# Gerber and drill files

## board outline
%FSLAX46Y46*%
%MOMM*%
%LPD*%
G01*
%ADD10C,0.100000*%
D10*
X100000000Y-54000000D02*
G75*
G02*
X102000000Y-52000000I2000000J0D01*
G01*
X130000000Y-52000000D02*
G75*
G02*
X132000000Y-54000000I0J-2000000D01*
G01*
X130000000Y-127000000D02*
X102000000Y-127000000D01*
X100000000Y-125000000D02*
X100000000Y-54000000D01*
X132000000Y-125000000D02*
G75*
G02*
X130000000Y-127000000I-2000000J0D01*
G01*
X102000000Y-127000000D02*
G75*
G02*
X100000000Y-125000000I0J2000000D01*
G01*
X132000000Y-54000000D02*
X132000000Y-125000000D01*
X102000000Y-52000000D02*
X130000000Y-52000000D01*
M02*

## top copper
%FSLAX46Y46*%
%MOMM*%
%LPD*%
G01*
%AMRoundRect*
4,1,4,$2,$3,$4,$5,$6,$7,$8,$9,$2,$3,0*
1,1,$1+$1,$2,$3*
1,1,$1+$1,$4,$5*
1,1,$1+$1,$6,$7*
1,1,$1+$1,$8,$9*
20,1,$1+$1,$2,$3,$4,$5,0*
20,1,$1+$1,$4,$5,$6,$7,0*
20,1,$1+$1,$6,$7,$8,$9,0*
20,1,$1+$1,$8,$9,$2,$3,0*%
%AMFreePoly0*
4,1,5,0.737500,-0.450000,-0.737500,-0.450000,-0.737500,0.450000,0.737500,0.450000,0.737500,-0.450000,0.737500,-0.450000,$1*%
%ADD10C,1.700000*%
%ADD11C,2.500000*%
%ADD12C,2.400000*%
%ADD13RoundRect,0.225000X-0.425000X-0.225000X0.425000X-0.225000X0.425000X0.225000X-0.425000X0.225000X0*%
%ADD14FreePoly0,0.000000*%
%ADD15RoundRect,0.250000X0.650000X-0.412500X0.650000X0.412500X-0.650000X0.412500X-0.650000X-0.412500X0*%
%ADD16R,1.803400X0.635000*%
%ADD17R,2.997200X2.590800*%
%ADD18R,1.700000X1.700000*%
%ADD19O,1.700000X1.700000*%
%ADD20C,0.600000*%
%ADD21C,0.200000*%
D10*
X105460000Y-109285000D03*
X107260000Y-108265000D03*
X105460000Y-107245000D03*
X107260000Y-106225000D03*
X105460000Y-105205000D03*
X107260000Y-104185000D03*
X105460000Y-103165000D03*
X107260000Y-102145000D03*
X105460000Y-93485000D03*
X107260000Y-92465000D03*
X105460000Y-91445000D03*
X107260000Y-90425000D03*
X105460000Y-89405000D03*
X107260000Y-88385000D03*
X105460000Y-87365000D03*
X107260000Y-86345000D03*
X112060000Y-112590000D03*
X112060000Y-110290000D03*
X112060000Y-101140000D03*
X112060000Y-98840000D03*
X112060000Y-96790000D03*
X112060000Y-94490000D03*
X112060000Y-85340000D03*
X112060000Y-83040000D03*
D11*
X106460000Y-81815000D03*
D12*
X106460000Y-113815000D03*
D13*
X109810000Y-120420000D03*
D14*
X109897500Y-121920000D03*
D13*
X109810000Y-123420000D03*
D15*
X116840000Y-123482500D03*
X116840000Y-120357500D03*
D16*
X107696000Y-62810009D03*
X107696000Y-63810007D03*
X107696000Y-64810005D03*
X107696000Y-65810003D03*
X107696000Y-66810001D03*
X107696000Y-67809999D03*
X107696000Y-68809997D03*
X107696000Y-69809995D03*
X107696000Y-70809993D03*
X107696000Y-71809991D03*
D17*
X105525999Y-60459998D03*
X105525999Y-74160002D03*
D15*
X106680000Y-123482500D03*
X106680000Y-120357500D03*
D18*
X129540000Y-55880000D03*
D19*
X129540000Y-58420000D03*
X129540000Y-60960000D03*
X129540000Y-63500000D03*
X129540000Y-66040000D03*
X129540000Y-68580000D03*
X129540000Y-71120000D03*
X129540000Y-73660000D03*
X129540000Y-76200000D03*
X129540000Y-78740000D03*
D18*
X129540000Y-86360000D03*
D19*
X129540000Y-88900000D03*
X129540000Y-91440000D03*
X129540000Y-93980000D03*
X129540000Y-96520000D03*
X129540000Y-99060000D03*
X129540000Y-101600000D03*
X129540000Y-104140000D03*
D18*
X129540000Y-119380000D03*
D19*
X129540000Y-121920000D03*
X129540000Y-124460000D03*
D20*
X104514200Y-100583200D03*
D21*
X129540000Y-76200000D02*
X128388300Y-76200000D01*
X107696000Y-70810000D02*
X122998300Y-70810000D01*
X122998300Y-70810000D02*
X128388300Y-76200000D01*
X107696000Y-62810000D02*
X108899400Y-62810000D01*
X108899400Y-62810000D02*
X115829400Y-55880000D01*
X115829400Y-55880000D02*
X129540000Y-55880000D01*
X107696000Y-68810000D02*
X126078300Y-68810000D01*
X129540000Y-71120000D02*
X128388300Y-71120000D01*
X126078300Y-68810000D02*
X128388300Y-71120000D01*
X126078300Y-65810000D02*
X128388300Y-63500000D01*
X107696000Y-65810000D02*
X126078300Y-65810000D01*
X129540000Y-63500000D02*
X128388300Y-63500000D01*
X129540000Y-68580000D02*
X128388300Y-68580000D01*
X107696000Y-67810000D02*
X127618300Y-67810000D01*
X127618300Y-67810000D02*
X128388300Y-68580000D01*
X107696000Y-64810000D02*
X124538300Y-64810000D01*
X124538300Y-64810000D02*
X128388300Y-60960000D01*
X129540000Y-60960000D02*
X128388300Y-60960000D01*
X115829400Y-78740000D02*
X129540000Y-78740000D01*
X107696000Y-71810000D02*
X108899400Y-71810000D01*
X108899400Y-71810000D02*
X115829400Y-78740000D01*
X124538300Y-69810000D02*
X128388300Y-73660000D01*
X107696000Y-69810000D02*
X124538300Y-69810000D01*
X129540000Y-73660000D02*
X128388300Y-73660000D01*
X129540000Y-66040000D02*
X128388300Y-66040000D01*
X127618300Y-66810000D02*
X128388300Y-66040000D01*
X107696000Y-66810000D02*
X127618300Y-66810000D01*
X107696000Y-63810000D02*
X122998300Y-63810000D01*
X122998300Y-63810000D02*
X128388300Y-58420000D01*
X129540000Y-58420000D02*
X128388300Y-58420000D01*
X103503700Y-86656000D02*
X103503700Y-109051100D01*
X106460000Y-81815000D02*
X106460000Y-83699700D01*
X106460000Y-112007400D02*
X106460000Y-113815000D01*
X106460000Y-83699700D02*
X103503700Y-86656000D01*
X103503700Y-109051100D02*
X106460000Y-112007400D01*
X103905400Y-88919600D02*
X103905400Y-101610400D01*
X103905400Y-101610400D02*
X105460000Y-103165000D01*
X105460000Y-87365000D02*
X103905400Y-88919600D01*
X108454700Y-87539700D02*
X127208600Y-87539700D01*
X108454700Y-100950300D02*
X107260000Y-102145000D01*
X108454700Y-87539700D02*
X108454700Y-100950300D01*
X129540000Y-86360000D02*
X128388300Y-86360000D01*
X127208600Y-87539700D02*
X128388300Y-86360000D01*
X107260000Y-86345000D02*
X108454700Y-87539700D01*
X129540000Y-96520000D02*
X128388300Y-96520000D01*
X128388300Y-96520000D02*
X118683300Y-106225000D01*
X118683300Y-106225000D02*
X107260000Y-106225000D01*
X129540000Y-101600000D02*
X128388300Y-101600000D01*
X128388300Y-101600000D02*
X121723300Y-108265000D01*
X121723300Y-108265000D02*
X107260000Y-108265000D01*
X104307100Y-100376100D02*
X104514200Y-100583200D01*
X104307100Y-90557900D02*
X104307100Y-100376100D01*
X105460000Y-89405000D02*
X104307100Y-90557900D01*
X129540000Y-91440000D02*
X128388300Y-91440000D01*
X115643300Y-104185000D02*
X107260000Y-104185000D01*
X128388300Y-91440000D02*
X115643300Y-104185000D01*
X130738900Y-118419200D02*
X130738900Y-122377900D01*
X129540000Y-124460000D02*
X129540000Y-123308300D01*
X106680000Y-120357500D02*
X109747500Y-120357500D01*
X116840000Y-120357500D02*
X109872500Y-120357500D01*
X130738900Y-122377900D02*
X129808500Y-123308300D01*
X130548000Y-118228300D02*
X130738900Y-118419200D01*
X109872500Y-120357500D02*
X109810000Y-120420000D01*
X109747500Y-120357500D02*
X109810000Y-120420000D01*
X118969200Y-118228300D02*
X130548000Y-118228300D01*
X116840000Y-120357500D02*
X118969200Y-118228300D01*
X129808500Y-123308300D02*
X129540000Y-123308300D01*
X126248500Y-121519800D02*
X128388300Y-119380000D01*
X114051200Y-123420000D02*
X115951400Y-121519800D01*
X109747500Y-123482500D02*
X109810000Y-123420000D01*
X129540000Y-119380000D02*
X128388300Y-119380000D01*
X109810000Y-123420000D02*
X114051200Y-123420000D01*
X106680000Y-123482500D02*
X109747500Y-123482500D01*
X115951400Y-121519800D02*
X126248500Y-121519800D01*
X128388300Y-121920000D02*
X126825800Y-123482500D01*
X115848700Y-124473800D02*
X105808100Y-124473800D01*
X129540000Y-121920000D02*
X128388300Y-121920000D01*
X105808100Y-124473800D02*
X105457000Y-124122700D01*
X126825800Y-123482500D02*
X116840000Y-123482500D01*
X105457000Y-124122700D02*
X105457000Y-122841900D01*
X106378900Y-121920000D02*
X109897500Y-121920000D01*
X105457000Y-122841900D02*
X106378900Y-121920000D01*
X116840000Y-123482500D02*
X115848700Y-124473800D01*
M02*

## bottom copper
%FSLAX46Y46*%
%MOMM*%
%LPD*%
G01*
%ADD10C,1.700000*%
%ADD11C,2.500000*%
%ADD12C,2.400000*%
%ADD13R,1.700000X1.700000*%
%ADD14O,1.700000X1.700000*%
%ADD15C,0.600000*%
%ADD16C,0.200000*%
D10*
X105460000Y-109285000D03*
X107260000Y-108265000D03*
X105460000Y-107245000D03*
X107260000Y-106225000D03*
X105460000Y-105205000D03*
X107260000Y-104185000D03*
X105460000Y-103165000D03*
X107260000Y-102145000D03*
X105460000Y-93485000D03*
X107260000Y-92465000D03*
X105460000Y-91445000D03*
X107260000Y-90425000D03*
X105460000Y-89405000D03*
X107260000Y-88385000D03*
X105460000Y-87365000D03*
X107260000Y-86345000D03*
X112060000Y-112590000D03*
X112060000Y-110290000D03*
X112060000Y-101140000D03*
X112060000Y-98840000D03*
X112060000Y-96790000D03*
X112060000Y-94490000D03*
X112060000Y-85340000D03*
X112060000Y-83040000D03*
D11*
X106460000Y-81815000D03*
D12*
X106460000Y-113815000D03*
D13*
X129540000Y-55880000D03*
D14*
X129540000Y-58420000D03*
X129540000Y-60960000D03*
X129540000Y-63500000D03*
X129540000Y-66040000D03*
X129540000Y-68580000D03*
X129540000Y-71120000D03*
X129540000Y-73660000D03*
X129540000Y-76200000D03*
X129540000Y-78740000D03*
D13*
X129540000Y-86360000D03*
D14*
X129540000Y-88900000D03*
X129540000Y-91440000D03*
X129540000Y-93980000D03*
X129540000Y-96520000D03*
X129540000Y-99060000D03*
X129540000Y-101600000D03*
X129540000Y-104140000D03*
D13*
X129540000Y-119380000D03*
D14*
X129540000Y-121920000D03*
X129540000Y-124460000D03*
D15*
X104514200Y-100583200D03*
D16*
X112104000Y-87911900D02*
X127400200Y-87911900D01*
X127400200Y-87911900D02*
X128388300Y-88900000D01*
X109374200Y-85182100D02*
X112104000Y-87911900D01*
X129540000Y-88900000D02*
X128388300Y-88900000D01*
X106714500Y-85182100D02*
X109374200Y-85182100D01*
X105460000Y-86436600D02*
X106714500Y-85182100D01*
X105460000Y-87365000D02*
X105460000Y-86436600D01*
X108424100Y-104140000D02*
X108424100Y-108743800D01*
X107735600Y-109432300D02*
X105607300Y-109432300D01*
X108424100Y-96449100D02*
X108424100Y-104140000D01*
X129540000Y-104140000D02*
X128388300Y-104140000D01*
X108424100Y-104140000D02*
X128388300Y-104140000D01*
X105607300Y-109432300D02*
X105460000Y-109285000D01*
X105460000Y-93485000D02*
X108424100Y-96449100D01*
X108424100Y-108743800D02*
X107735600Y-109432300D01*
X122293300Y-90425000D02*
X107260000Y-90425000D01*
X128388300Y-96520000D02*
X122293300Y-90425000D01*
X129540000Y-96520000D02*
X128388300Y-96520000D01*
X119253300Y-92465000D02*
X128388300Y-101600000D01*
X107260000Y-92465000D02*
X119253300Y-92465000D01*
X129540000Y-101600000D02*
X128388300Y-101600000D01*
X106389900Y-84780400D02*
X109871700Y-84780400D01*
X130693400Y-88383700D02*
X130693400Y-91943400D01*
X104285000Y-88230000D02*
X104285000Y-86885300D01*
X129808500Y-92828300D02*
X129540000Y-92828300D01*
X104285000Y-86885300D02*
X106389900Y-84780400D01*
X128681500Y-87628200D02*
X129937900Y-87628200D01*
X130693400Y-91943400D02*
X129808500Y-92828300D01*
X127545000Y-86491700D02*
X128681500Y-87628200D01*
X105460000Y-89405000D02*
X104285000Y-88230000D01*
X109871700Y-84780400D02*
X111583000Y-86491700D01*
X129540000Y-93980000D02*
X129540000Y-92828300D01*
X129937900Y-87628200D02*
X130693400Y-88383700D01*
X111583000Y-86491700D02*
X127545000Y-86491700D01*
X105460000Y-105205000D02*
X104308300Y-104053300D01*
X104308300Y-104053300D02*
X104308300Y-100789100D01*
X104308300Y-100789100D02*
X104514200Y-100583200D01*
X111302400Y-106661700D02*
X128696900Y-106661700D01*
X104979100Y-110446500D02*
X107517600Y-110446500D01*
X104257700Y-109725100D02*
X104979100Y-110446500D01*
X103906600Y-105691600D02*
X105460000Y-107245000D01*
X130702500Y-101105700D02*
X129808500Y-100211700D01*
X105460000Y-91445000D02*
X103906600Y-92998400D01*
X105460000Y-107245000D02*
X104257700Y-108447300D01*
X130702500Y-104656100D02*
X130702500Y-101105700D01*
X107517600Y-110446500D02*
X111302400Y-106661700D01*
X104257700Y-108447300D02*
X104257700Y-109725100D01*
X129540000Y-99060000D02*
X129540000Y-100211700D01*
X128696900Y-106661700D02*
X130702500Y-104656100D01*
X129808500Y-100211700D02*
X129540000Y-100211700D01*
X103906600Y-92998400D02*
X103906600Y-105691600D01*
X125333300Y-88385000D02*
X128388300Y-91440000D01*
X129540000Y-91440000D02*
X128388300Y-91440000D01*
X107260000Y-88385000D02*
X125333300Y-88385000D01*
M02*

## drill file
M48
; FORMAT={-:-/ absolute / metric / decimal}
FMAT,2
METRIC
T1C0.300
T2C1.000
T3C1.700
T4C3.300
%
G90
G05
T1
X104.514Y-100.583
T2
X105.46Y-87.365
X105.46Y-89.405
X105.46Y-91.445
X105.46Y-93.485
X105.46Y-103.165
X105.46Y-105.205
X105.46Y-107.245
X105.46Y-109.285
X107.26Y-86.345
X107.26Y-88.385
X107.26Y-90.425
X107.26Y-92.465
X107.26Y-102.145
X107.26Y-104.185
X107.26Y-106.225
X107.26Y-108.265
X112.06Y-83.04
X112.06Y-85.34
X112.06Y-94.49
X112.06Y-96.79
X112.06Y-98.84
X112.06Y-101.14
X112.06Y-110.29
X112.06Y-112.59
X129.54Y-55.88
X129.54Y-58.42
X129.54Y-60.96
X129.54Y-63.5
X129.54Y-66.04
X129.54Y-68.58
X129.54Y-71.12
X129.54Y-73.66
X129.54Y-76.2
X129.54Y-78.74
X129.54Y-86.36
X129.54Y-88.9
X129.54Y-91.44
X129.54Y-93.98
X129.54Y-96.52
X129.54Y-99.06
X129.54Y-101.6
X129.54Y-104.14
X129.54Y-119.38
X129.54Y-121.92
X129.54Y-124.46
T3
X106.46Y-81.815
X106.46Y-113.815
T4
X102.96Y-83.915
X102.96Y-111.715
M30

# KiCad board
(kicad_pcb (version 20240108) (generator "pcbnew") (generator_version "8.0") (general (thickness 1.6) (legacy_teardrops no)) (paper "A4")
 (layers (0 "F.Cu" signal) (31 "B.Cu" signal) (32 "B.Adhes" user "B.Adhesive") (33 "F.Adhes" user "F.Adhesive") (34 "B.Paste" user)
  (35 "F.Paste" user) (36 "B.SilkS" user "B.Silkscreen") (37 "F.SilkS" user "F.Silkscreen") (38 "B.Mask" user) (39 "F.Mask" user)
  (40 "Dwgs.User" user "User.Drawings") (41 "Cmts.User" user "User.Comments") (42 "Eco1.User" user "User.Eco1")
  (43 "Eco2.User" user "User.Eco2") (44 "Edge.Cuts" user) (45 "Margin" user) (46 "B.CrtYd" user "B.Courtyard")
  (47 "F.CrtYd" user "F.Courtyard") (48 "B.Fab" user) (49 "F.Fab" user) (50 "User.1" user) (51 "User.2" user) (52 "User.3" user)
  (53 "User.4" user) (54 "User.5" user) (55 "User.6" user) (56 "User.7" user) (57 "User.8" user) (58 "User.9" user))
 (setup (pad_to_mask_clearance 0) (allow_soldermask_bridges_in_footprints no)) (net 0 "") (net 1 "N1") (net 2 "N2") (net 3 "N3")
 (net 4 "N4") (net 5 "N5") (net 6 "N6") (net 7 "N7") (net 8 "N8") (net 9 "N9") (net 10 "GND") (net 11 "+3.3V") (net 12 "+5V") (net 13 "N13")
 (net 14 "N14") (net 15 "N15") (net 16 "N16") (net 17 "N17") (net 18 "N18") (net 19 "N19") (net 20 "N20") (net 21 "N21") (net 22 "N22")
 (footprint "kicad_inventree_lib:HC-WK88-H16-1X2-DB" (layer "F.Cu") (at 110.54 93.485 -90)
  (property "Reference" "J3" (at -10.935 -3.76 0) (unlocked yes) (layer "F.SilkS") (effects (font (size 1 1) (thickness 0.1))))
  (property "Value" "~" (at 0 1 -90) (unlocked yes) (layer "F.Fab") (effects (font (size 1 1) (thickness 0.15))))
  (pad "" np_thru_hole circle (at -9.57 7.58 270) (size 1 1) (drill 3.3) (layers "F&B.Cu" "*.Mask"))
  (pad "" np_thru_hole circle (at 18.23 7.58 270) (size 1 1) (drill 3.3) (layers "F&B.Cu" "*.Mask"))
  (pad "1" thru_hole circle (at 15.8 5.08 270) (size 1.7 1.7) (drill 1) (layers "*.Cu" "*.Mask") (remove_unused_layers no) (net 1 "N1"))
  (pad "2" thru_hole circle (at 14.78 3.28 270) (size 1.7 1.7) (drill 1) (layers "*.Cu" "*.Mask") (remove_unused_layers no) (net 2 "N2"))
  (pad "3" thru_hole circle (at 13.76 5.08 270) (size 1.7 1.7) (drill 1) (layers "*.Cu" "*.Mask") (remove_unused_layers no) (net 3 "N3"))
  (pad "4" thru_hole circle (at 12.74 3.28 270) (size 1.7 1.7) (drill 1) (layers "*.Cu" "*.Mask") (remove_unused_layers no) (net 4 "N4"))
  (pad "5" thru_hole circle (at 11.72 5.08 270) (size 1.7 1.7) (drill 1) (layers "*.Cu" "*.Mask") (remove_unused_layers no) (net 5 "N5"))
  (pad "6" thru_hole circle (at 10.7 3.28 270) (size 1.7 1.7) (drill 1) (layers "*.Cu" "*.Mask") (remove_unused_layers no) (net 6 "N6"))
  (pad "7" thru_hole circle (at 9.68 5.08 270) (size 1.7 1.7) (drill 1) (layers "*.Cu" "*.Mask") (remove_unused_layers no) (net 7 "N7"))
  (pad "8" thru_hole circle (at 8.66 3.28 270) (size 1.7 1.7) (drill 1) (layers "*.Cu" "*.Mask") (remove_unused_layers no) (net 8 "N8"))
  (pad "9" thru_hole circle (at 0 5.08 270) (size 1.7 1.7) (drill 1) (layers "*.Cu" "*.Mask") (remove_unused_layers no) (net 1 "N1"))
  (pad "10" thru_hole circle (at -1.02 3.28 270) (size 1.7 1.7) (drill 1) (layers "*.Cu" "*.Mask") (remove_unused_layers no) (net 2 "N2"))
  (pad "11" thru_hole circle (at -2.04 5.08 270) (size 1.7 1.7) (drill 1) (layers "*.Cu" "*.Mask") (remove_unused_layers no) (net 3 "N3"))
  (pad "12" thru_hole circle (at -3.06 3.28 270) (size 1.7 1.7) (drill 1) (layers "*.Cu" "*.Mask") (remove_unused_layers no) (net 4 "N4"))
  (pad "13" thru_hole circle (at -4.08 5.08 270) (size 1.7 1.7) (drill 1) (layers "*.Cu" "*.Mask") (remove_unused_layers no) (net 5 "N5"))
  (pad "14" thru_hole circle (at -5.1 3.28 270) (size 1.7 1.7) (drill 1) (layers "*.Cu" "*.Mask") (remove_unused_layers no) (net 6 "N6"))
  (pad "15" thru_hole circle (at -6.12 5.08 270) (size 1.7 1.7) (drill 1) (layers "*.Cu" "*.Mask") (remove_unused_layers no) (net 7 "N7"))
  (pad "16" thru_hole circle (at -7.14 3.28 270) (size 1.7 1.7) (drill 1) (layers "*.Cu" "*.Mask") (remove_unused_layers no) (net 8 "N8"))
  (pad "17" thru_hole circle (at 19.105 -1.52 270) (size 1.7 1.7) (drill 1) (layers "*.Cu" "*.Mask") (remove_unused_layers no))
  (pad "18" thru_hole circle (at 16.805 -1.52 270) (size 1.7 1.7) (drill 1) (layers "*.Cu" "*.Mask") (remove_unused_layers no))
  (pad "19" thru_hole circle (at 7.655 -1.52 270) (size 1.7 1.7) (drill 1) (layers "*.Cu" "*.Mask") (remove_unused_layers no))
  (pad "20" thru_hole circle (at 5.355 -1.52 270) (size 1.7 1.7) (drill 1) (layers "*.Cu" "*.Mask") (remove_unused_layers no))
  (pad "21" thru_hole circle (at 3.305 -1.52 270) (size 1.7 1.7) (drill 1) (layers "*.Cu" "*.Mask") (remove_unused_layers no))
  (pad "22" thru_hole circle (at 1.005 -1.52 270) (size 1.7 1.7) (drill 1) (layers "*.Cu" "*.Mask") (remove_unused_layers no))
  (pad "23" thru_hole circle (at -8.145 -1.52 270) (size 1.7 1.7) (drill 1) (layers "*.Cu" "*.Mask") (remove_unused_layers no))
  (pad "24" thru_hole circle (at -10.445 -1.52 270) (size 1.7 1.7) (drill 1) (layers "*.Cu" "*.Mask") (remove_unused_layers no))
  (pad "PE" thru_hole circle (at -11.67 4.08 270) (size 2.5 2.5) (drill 1.7) (layers "*.Cu" "*.Mask") (remove_unused_layers no) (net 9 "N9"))
  (pad "PE" thru_hole circle (at 20.33 4.08 270) (size 2.4 2.4) (drill 1.7) (layers "*.Cu" "*.Mask") (remove_unused_layers no) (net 9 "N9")))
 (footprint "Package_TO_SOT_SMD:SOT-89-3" (layer "F.Cu") (at 111.76 121.92)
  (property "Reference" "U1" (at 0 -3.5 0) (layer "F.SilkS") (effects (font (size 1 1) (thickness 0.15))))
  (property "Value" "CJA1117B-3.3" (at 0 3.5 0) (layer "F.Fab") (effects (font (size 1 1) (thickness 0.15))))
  (pad "1" smd roundrect (at -1.95 -1.5) (size 1.3 0.9) (layers "F.Cu" "F.Paste" "F.Mask") (roundrect_rratio 0.25) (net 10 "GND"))
  (pad "2" smd custom (at -1.8625 0) (size 1.475 0.9) (layers "F.Cu" "F.Paste" "F.Mask") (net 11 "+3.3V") (zone_connect 2)
   (thermal_bridge_angle 45) (options (clearance outline) (anchor rect)) (primitives))
  (pad "3" smd roundrect (at -1.95 1.5) (size 1.3 0.9) (layers "F.Cu" "F.Paste" "F.Mask") (roundrect_rratio 0.25) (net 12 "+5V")))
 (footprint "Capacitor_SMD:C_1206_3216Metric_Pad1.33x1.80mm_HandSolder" (layer "F.Cu") (at 116.84 121.92 90)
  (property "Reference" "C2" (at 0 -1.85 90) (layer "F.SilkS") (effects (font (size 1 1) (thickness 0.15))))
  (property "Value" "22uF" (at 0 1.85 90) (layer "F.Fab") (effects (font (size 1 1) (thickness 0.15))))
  (pad "1" smd roundrect (at -1.5625 0 90) (size 1.325 1.8) (layers "F.Cu" "F.Paste" "F.Mask") (roundrect_rratio 0.188679) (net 11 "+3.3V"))
  (pad "2" smd roundrect (at 1.5625 0 90) (size 1.325 1.8) (layers "F.Cu" "F.Paste" "F.Mask") (roundrect_rratio 0.188679) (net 10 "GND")))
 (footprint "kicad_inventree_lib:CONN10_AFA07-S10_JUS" (layer "F.Cu") (at 104.14 67.31 -90)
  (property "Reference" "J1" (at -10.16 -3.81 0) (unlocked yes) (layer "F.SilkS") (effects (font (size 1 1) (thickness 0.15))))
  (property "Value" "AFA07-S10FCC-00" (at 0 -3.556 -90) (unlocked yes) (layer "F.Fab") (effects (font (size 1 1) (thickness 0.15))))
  (pad "1" smd rect (at -4.499991 -3.556 270) (size 0.635 1.8034) (layers "F.Cu" "F.Paste" "F.Mask") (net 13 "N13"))
  (pad "2" smd rect (at -3.499993 -3.556 270) (size 0.635 1.8034) (layers "F.Cu" "F.Paste" "F.Mask") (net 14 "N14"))
  (pad "3" smd rect (at -2.499995 -3.556 270) (size 0.635 1.8034) (layers "F.Cu" "F.Paste" "F.Mask") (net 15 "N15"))
  (pad "4" smd rect (at -1.499997 -3.556 270) (size 0.635 1.8034) (layers "F.Cu" "F.Paste" "F.Mask") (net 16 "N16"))
  (pad "5" smd rect (at -0.499999 -3.556 270) (size 0.635 1.8034) (layers "F.Cu" "F.Paste" "F.Mask") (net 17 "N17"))
  (pad "6" smd rect (at 0.499999 -3.556 270) (size 0.635 1.8034) (layers "F.Cu" "F.Paste" "F.Mask") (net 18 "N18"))
  (pad "7" smd rect (at 1.499997 -3.556 270) (size 0.635 1.8034) (layers "F.Cu" "F.Paste" "F.Mask") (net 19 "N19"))
  (pad "8" smd rect (at 2.499995 -3.556 270) (size 0.635 1.8034) (layers "F.Cu" "F.Paste" "F.Mask") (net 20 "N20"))
  (pad "9" smd rect (at 3.499993 -3.556 270) (size 0.635 1.8034) (layers "F.Cu" "F.Paste" "F.Mask") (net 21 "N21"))
  (pad "10" smd rect (at 4.499991 -3.556 270) (size 0.635 1.8034) (layers "F.Cu" "F.Paste" "F.Mask") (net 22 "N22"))
  (pad "11" smd rect (at -6.850002 -1.385999 270) (size 2.5908 2.9972) (layers "F.Cu" "F.Paste" "F.Mask"))
  (pad "12" smd rect (at 6.850002 -1.385999 270) (size 2.5908 2.9972) (layers "F.Cu" "F.Paste" "F.Mask")))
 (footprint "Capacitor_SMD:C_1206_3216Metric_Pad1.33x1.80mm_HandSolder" (layer "F.Cu") (at 106.68 121.92 90)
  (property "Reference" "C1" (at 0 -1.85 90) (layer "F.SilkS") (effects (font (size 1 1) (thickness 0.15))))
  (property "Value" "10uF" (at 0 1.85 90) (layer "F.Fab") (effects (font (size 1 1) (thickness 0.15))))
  (pad "1" smd roundrect (at -1.5625 0 90) (size 1.325 1.8) (layers "F.Cu" "F.Paste" "F.Mask") (roundrect_rratio 0.188679) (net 12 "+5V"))
  (pad "2" smd roundrect (at 1.5625 0 90) (size 1.325 1.8) (layers "F.Cu" "F.Paste" "F.Mask") (roundrect_rratio 0.188679) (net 10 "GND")))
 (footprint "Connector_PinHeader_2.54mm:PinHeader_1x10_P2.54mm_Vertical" (layer "B.Cu") (at 129.54 55.88 180)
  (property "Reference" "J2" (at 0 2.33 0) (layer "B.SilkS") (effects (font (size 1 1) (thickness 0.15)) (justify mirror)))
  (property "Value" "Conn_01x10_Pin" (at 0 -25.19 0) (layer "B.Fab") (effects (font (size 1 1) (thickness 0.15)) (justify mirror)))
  (pad "1" thru_hole rect (at 0 0 180) (size 1.7 1.7) (drill 1) (layers "*.Cu" "*.Mask") (remove_unused_layers no) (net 13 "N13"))
  (pad "2" thru_hole oval (at 0 -2.54 180) (size 1.7 1.7) (drill 1) (layers "*.Cu" "*.Mask") (remove_unused_layers no) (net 14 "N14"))
  (pad "3" thru_hole oval (at 0 -5.08 180) (size 1.7 1.7) (drill 1) (layers "*.Cu" "*.Mask") (remove_unused_layers no) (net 15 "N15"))
  (pad "4" thru_hole oval (at 0 -7.62 180) (size 1.7 1.7) (drill 1) (layers "*.Cu" "*.Mask") (remove_unused_layers no) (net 16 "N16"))
  (pad "5" thru_hole oval (at 0 -10.16 180) (size 1.7 1.7) (drill 1) (layers "*.Cu" "*.Mask") (remove_unused_layers no) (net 17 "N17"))
  (pad "6" thru_hole oval (at 0 -12.7 180) (size 1.7 1.7) (drill 1) (layers "*.Cu" "*.Mask") (remove_unused_layers no) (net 18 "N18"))
  (pad "7" thru_hole oval (at 0 -15.24 180) (size 1.7 1.7) (drill 1) (layers "*.Cu" "*.Mask") (remove_unused_layers no) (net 19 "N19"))
  (pad "8" thru_hole oval (at 0 -17.78 180) (size 1.7 1.7) (drill 1) (layers "*.Cu" "*.Mask") (remove_unused_layers no) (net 20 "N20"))
  (pad "9" thru_hole oval (at 0 -20.32 180) (size 1.7 1.7) (drill 1) (layers "*.Cu" "*.Mask") (remove_unused_layers no) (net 21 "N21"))
  (pad "10" thru_hole oval (at 0 -22.86 180) (size 1.7 1.7) (drill 1) (layers "*.Cu" "*.Mask") (remove_unused_layers no) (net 22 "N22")))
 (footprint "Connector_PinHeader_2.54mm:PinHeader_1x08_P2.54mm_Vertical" (layer "B.Cu") (at 129.54 86.36 180)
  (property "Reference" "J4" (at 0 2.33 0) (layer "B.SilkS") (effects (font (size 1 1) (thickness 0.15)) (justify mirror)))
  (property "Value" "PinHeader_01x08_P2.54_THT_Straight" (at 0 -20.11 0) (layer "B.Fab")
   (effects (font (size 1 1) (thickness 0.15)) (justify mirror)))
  (pad "1" thru_hole rect (at 0 0 180) (size 1.7 1.7) (drill 1) (layers "*.Cu" "*.Mask") (remove_unused_layers no) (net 8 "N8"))
  (pad "2" thru_hole oval (at 0 -2.54 180) (size 1.7 1.7) (drill 1) (layers "*.Cu" "*.Mask") (remove_unused_layers no) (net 7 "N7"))
  (pad "3" thru_hole oval (at 0 -5.08 180) (size 1.7 1.7) (drill 1) (layers "*.Cu" "*.Mask") (remove_unused_layers no) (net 6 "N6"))
  (pad "4" thru_hole oval (at 0 -7.62 180) (size 1.7 1.7) (drill 1) (layers "*.Cu" "*.Mask") (remove_unused_layers no) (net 5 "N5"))
  (pad "5" thru_hole oval (at 0 -10.16 180) (size 1.7 1.7) (drill 1) (layers "*.Cu" "*.Mask") (remove_unused_layers no) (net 4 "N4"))
  (pad "6" thru_hole oval (at 0 -12.7 180) (size 1.7 1.7) (drill 1) (layers "*.Cu" "*.Mask") (remove_unused_layers no) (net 3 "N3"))
  (pad "7" thru_hole oval (at 0 -15.24 180) (size 1.7 1.7) (drill 1) (layers "*.Cu" "*.Mask") (remove_unused_layers no) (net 2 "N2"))
  (pad "8" thru_hole oval (at 0 -17.78 180) (size 1.7 1.7) (drill 1) (layers "*.Cu" "*.Mask") (remove_unused_layers no) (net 1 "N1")))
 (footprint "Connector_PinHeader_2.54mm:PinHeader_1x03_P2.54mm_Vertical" (layer "B.Cu") (at 129.54 119.38 180)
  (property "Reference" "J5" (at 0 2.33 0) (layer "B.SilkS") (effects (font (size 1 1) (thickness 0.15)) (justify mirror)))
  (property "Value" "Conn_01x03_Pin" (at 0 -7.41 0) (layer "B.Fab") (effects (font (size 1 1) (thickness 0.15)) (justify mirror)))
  (pad "1" thru_hole rect (at 0 0 180) (size 1.7 1.7) (drill 1) (layers "*.Cu" "*.Mask") (remove_unused_layers no) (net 12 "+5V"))
  (pad "2" thru_hole oval (at 0 -2.54 180) (size 1.7 1.7) (drill 1) (layers "*.Cu" "*.Mask") (remove_unused_layers no) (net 11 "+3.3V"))
  (pad "3" thru_hole oval (at 0 -5.08 180) (size 1.7 1.7) (drill 1) (layers "*.Cu" "*.Mask") (remove_unused_layers no) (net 10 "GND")))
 (gr_arc (start 100 54) (mid 100.585786 52.585786) (end 102 52) (stroke (width 0.1) (type default)) (layer "Edge.Cuts"))
 (gr_arc (start 130 52) (mid 131.414214 52.585786) (end 132 54) (stroke (width 0.1) (type default)) (layer "Edge.Cuts"))
 (gr_line (start 130 127) (end 102 127) (stroke (width 0.1) (type default)) (layer "Edge.Cuts"))
 (gr_line (start 100 125) (end 100 54) (stroke (width 0.1) (type default)) (layer "Edge.Cuts"))
 (gr_arc (start 132 125) (mid 131.414214 126.414214) (end 130 127) (stroke (width 0.1) (type default)) (layer "Edge.Cuts"))
 (gr_arc (start 102 127) (mid 100.585786 126.414214) (end 100 125) (stroke (width 0.1) (type default)) (layer "Edge.Cuts"))
 (gr_line (start 132 54) (end 132 125) (stroke (width 0.1) (type default)) (layer "Edge.Cuts"))
 (gr_line (start 102 52) (end 130 52) (stroke (width 0.1) (type default)) (layer "Edge.Cuts"))
 (segment (start 129.54 76.2) (end 128.3883 76.2) (width 0.2) (layer "F.Cu") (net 21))
 (segment (start 107.696 70.81) (end 122.9983 70.81) (width 0.2) (layer "F.Cu") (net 21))
 (segment (start 122.9983 70.81) (end 128.3883 76.2) (width 0.2) (layer "F.Cu") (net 21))
 (segment (start 107.696 62.81) (end 108.8994 62.81) (width 0.2) (layer "F.Cu") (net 13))
 (segment (start 108.8994 62.81) (end 115.8294 55.88) (width 0.2) (layer "F.Cu") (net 13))
 (segment (start 115.8294 55.88) (end 129.54 55.88) (width 0.2) (layer "F.Cu") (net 13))
 (segment (start 107.696 68.81) (end 126.0783 68.81) (width 0.2) (layer "F.Cu") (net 19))
 (segment (start 129.54 71.12) (end 128.3883 71.12) (width 0.2) (layer "F.Cu") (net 19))
 (segment (start 126.0783 68.81) (end 128.3883 71.12) (width 0.2) (layer "F.Cu") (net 19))
 (segment (start 126.0783 65.81) (end 128.3883 63.5) (width 0.2) (layer "F.Cu") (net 16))
 (segment (start 107.696 65.81) (end 126.0783 65.81) (width 0.2) (layer "F.Cu") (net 16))
 (segment (start 129.54 63.5) (end 128.3883 63.5) (width 0.2) (layer "F.Cu") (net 16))
 (segment (start 129.54 68.58) (end 128.3883 68.58) (width 0.2) (layer "F.Cu") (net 18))
 (segment (start 107.696 67.81) (end 127.6183 67.81) (width 0.2) (layer "F.Cu") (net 18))
 (segment (start 127.6183 67.81) (end 128.3883 68.58) (width 0.2) (layer "F.Cu") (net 18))
 (segment (start 107.696 64.81) (end 124.5383 64.81) (width 0.2) (layer "F.Cu") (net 15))
 (segment (start 124.5383 64.81) (end 128.3883 60.96) (width 0.2) (layer "F.Cu") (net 15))
 (segment (start 129.54 60.96) (end 128.3883 60.96) (width 0.2) (layer "F.Cu") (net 15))
 (segment (start 115.8294 78.74) (end 129.54 78.74) (width 0.2) (layer "F.Cu") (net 22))
 (segment (start 107.696 71.81) (end 108.8994 71.81) (width 0.2) (layer "F.Cu") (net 22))
 (segment (start 108.8994 71.81) (end 115.8294 78.74) (width 0.2) (layer "F.Cu") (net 22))
 (segment (start 124.5383 69.81) (end 128.3883 73.66) (width 0.2) (layer "F.Cu") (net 20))
 (segment (start 107.696 69.81) (end 124.5383 69.81) (width 0.2) (layer "F.Cu") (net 20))
 (segment (start 129.54 73.66) (end 128.3883 73.66) (width 0.2) (layer "F.Cu") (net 20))
 (segment (start 129.54 66.04) (end 128.3883 66.04) (width 0.2) (layer "F.Cu") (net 17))
 (segment (start 127.6183 66.81) (end 128.3883 66.04) (width 0.2) (layer "F.Cu") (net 17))
 (segment (start 107.696 66.81) (end 127.6183 66.81) (width 0.2) (layer "F.Cu") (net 17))
 (segment (start 107.696 63.81) (end 122.9983 63.81) (width 0.2) (layer "F.Cu") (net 14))
 (segment (start 122.9983 63.81) (end 128.3883 58.42) (width 0.2) (layer "F.Cu") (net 14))
 (segment (start 129.54 58.42) (end 128.3883 58.42) (width 0.2) (layer "F.Cu") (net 14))
 (segment (start 103.5037 86.656) (end 103.5037 109.0511) (width 0.2) (layer "F.Cu") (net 9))
 (segment (start 106.46 81.815) (end 106.46 83.6997) (width 0.2) (layer "F.Cu") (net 9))
 (segment (start 106.46 112.0074) (end 106.46 113.815) (width 0.2) (layer "F.Cu") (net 9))
 (segment (start 106.46 83.6997) (end 103.5037 86.656) (width 0.2) (layer "F.Cu") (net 9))
 (segment (start 103.5037 109.0511) (end 106.46 112.0074) (width 0.2) (layer "F.Cu") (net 9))
 (segment (start 103.9054 88.9196) (end 103.9054 101.6104) (width 0.2) (layer "F.Cu") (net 7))
 (segment (start 103.9054 101.6104) (end 105.46 103.165) (width 0.2) (layer "F.Cu") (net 7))
 (segment (start 105.46 87.365) (end 103.9054 88.9196) (width 0.2) (layer "F.Cu") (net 7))
 (segment (start 112.104 87.9119) (end 127.4002 87.9119) (width 0.2) (layer "B.Cu") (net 7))
 (segment (start 127.4002 87.9119) (end 128.3883 88.9) (width 0.2) (layer "B.Cu") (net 7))
 (segment (start 109.3742 85.1821) (end 112.104 87.9119) (width 0.2) (layer "B.Cu") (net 7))
 (segment (start 129.54 88.9) (end 128.3883 88.9) (width 0.2) (layer "B.Cu") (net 7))
 (segment (start 106.7145 85.1821) (end 109.3742 85.1821) (width 0.2) (layer "B.Cu") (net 7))
 (segment (start 105.46 86.4366) (end 106.7145 85.1821) (width 0.2) (layer "B.Cu") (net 7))
 (segment (start 105.46 87.365) (end 105.46 86.4366) (width 0.2) (layer "B.Cu") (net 7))
 (segment (start 108.4547 87.5397) (end 127.2086 87.5397) (width 0.2) (layer "F.Cu") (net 8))
 (segment (start 108.4547 100.9503) (end 107.26 102.145) (width 0.2) (layer "F.Cu") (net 8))
 (segment (start 108.4547 87.5397) (end 108.4547 100.9503) (width 0.2) (layer "F.Cu") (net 8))
 (segment (start 129.54 86.36) (end 128.3883 86.36) (width 0.2) (layer "F.Cu") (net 8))
 (segment (start 127.2086 87.5397) (end 128.3883 86.36) (width 0.2) (layer "F.Cu") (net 8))
 (segment (start 107.26 86.345) (end 108.4547 87.5397) (width 0.2) (layer "F.Cu") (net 8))
 (segment (start 108.4241 104.14) (end 108.4241 108.7438) (width 0.2) (layer "B.Cu") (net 1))
 (segment (start 107.7356 109.4323) (end 105.6073 109.4323) (width 0.2) (layer "B.Cu") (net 1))
 (segment (start 108.4241 96.4491) (end 108.4241 104.14) (width 0.2) (layer "B.Cu") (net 1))
 (segment (start 129.54 104.14) (end 128.3883 104.14) (width 0.2) (layer "B.Cu") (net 1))
 (segment (start 108.4241 104.14) (end 128.3883 104.14) (width 0.2) (layer "B.Cu") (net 1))
 (segment (start 105.6073 109.4323) (end 105.46 109.285) (width 0.2) (layer "B.Cu") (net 1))
 (segment (start 105.46 93.485) (end 108.4241 96.4491) (width 0.2) (layer "B.Cu") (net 1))
 (segment (start 108.4241 108.7438) (end 107.7356 109.4323) (width 0.2) (layer "B.Cu") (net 1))
 (segment (start 129.54 96.52) (end 128.3883 96.52) (width 0.2) (layer "F.Cu") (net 4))
 (segment (start 128.3883 96.52) (end 118.6833 106.225) (width 0.2) (layer "F.Cu") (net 4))
 (segment (start 118.6833 106.225) (end 107.26 106.225) (width 0.2) (layer "F.Cu") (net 4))
 (segment (start 122.2933 90.425) (end 107.26 90.425) (width 0.2) (layer "B.Cu") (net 4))
 (segment (start 128.3883 96.52) (end 122.2933 90.425) (width 0.2) (layer "B.Cu") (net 4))
 (segment (start 129.54 96.52) (end 128.3883 96.52) (width 0.2) (layer "B.Cu") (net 4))
 (segment (start 129.54 101.6) (end 128.3883 101.6) (width 0.2) (layer "F.Cu") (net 2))
 (segment (start 128.3883 101.6) (end 121.7233 108.265) (width 0.2) (layer "F.Cu") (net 2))
 (segment (start 121.7233 108.265) (end 107.26 108.265) (width 0.2) (layer "F.Cu") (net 2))
 (segment (start 119.2533 92.465) (end 128.3883 101.6) (width 0.2) (layer "B.Cu") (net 2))
 (segment (start 107.26 92.465) (end 119.2533 92.465) (width 0.2) (layer "B.Cu") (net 2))
 (segment (start 129.54 101.6) (end 128.3883 101.6) (width 0.2) (layer "B.Cu") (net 2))
 (segment (start 104.3071 100.3761) (end 104.5142 100.5832) (width 0.2) (layer "F.Cu") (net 5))
 (segment (start 104.3071 90.5579) (end 104.3071 100.3761) (width 0.2) (layer "F.Cu") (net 5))
 (segment (start 105.46 89.405) (end 104.3071 90.5579) (width 0.2) (layer "F.Cu") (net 5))
 (via (at 104.5142 100.5832) (size 0.6) (drill 0.3) (layers "F.Cu" "B.Cu") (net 5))
 (segment (start 106.3899 84.7804) (end 109.8717 84.7804) (width 0.2) (layer "B.Cu") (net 5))
 (segment (start 130.6934 88.3837) (end 130.6934 91.9434) (width 0.2) (layer "B.Cu") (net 5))
 (segment (start 104.285 88.23) (end 104.285 86.8853) (width 0.2) (layer "B.Cu") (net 5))
 (segment (start 129.8085 92.8283) (end 129.54 92.8283) (width 0.2) (layer "B.Cu") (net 5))
 (segment (start 104.285 86.8853) (end 106.3899 84.7804) (width 0.2) (layer "B.Cu") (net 5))
 (segment (start 128.6815 87.6282) (end 129.9379 87.6282) (width 0.2) (layer "B.Cu") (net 5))
 (segment (start 130.6934 91.9434) (end 129.8085 92.8283) (width 0.2) (layer "B.Cu") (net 5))
 (segment (start 127.545 86.4917) (end 128.6815 87.6282) (width 0.2) (layer "B.Cu") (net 5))
 (segment (start 105.46 89.405) (end 104.285 88.23) (width 0.2) (layer "B.Cu") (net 5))
 (segment (start 109.8717 84.7804) (end 111.583 86.4917) (width 0.2) (layer "B.Cu") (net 5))
 (segment (start 129.54 93.98) (end 129.54 92.8283) (width 0.2) (layer "B.Cu") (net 5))
 (segment (start 129.9379 87.6282) (end 130.6934 88.3837) (width 0.2) (layer "B.Cu") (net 5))
 (segment (start 111.583 86.4917) (end 127.545 86.4917) (width 0.2) (layer "B.Cu") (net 5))
 (segment (start 105.46 105.205) (end 104.3083 104.0533) (width 0.2) (layer "B.Cu") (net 5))
 (segment (start 104.3083 104.0533) (end 104.3083 100.7891) (width 0.2) (layer "B.Cu") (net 5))
 (segment (start 104.3083 100.7891) (end 104.5142 100.5832) (width 0.2) (layer "B.Cu") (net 5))
 (segment (start 111.3024 106.6617) (end 128.6969 106.6617) (width 0.2) (layer "B.Cu") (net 3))
 (segment (start 104.9791 110.4465) (end 107.5176 110.4465) (width 0.2) (layer "B.Cu") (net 3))
 (segment (start 104.2577 109.7251) (end 104.9791 110.4465) (width 0.2) (layer "B.Cu") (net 3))
 (segment (start 103.9066 105.6916) (end 105.46 107.245) (width 0.2) (layer "B.Cu") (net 3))
 (segment (start 130.7025 101.1057) (end 129.8085 100.2117) (width 0.2) (layer "B.Cu") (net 3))
 (segment (start 105.46 91.445) (end 103.9066 92.9984) (width 0.2) (layer "B.Cu") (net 3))
 (segment (start 105.46 107.245) (end 104.2577 108.4473) (width 0.2) (layer "B.Cu") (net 3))
 (segment (start 130.7025 104.6561) (end 130.7025 101.1057) (width 0.2) (layer "B.Cu") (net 3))
 (segment (start 107.5176 110.4465) (end 111.3024 106.6617) (width 0.2) (layer "B.Cu") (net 3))
 (segment (start 104.2577 108.4473) (end 104.2577 109.7251) (width 0.2) (layer "B.Cu") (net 3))
 (segment (start 129.54 99.06) (end 129.54 100.2117) (width 0.2) (layer "B.Cu") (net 3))
 (segment (start 128.6969 106.6617) (end 130.7025 104.6561) (width 0.2) (layer "B.Cu") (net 3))
 (segment (start 129.8085 100.2117) (end 129.54 100.2117) (width 0.2) (layer "B.Cu") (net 3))
 (segment (start 103.9066 92.9984) (end 103.9066 105.6916) (width 0.2) (layer "B.Cu") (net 3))
 (segment (start 129.54 91.44) (end 128.3883 91.44) (width 0.2) (layer "F.Cu") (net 6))
 (segment (start 115.6433 104.185) (end 107.26 104.185) (width 0.2) (layer "F.Cu") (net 6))
 (segment (start 128.3883 91.44) (end 115.6433 104.185) (width 0.2) (layer "F.Cu") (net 6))
 (segment (start 125.3333 88.385) (end 128.3883 91.44) (width 0.2) (layer "B.Cu") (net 6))
 (segment (start 129.54 91.44) (end 128.3883 91.44) (width 0.2) (layer "B.Cu") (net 6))
 (segment (start 107.26 88.385) (end 125.3333 88.385) (width 0.2) (layer "B.Cu") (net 6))
 (segment (start 130.7389 118.4192) (end 130.7389 122.3779) (width 0.2) (layer "F.Cu") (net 10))
 (segment (start 129.54 124.46) (end 129.54 123.3083) (width 0.2) (layer "F.Cu") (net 10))
 (segment (start 106.68 120.3575) (end 109.7475 120.3575) (width 0.2) (layer "F.Cu") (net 10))
 (segment (start 116.84 120.3575) (end 109.8725 120.3575) (width 0.2) (layer "F.Cu") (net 10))
 (segment (start 130.7389 122.3779) (end 129.8085 123.3083) (width 0.2) (layer "F.Cu") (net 10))
 (segment (start 130.548 118.2283) (end 130.7389 118.4192) (width 0.2) (layer "F.Cu") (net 10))
 (segment (start 109.8725 120.3575) (end 109.81 120.42) (width 0.2) (layer "F.Cu") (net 10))
 (segment (start 109.7475 120.3575) (end 109.81 120.42) (width 0.2) (layer "F.Cu") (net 10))
 (segment (start 118.9692 118.2283) (end 130.548 118.2283) (width 0.2) (layer "F.Cu") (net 10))
 (segment (start 116.84 120.3575) (end 118.9692 118.2283) (width 0.2) (layer "F.Cu") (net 10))
 (segment (start 129.8085 123.3083) (end 129.54 123.3083) (width 0.2) (layer "F.Cu") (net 10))
 (segment (start 126.2485 121.5198) (end 128.3883 119.38) (width 0.2) (layer "F.Cu") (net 12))
 (segment (start 114.0512 123.42) (end 115.9514 121.5198) (width 0.2) (layer "F.Cu") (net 12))
 (segment (start 109.7475 123.4825) (end 109.81 123.42) (width 0.2) (layer "F.Cu") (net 12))
 (segment (start 129.54 119.38) (end 128.3883 119.38) (width 0.2) (layer "F.Cu") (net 12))
 (segment (start 109.81 123.42) (end 114.0512 123.42) (width 0.2) (layer "F.Cu") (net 12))
 (segment (start 106.68 123.4825) (end 109.7475 123.4825) (width 0.2) (layer "F.Cu") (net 12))
 (segment (start 115.9514 121.5198) (end 126.2485 121.5198) (width 0.2) (layer "F.Cu") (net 12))
 (segment (start 128.3883 121.92) (end 126.8258 123.4825) (width 0.2) (layer "F.Cu") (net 11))
 (segment (start 115.8487 124.4738) (end 105.8081 124.4738) (width 0.2) (layer "F.Cu") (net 11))
 (segment (start 129.54 121.92) (end 128.3883 121.92) (width 0.2) (layer "F.Cu") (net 11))
 (segment (start 105.8081 124.4738) (end 105.457 124.1227) (width 0.2) (layer "F.Cu") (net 11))
 (segment (start 126.8258 123.4825) (end 116.84 123.4825) (width 0.2) (layer "F.Cu") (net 11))
 (segment (start 105.457 124.1227) (end 105.457 122.8419) (width 0.2) (layer "F.Cu") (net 11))
 (segment (start 106.3789 121.92) (end 109.8975 121.92) (width 0.2) (layer "F.Cu") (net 11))
 (segment (start 105.457 122.8419) (end 106.3789 121.92) (width 0.2) (layer "F.Cu") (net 11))
 (segment (start 116.84 123.4825) (end 115.8487 124.4738) (width 0.2) (layer "F.Cu") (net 11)))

